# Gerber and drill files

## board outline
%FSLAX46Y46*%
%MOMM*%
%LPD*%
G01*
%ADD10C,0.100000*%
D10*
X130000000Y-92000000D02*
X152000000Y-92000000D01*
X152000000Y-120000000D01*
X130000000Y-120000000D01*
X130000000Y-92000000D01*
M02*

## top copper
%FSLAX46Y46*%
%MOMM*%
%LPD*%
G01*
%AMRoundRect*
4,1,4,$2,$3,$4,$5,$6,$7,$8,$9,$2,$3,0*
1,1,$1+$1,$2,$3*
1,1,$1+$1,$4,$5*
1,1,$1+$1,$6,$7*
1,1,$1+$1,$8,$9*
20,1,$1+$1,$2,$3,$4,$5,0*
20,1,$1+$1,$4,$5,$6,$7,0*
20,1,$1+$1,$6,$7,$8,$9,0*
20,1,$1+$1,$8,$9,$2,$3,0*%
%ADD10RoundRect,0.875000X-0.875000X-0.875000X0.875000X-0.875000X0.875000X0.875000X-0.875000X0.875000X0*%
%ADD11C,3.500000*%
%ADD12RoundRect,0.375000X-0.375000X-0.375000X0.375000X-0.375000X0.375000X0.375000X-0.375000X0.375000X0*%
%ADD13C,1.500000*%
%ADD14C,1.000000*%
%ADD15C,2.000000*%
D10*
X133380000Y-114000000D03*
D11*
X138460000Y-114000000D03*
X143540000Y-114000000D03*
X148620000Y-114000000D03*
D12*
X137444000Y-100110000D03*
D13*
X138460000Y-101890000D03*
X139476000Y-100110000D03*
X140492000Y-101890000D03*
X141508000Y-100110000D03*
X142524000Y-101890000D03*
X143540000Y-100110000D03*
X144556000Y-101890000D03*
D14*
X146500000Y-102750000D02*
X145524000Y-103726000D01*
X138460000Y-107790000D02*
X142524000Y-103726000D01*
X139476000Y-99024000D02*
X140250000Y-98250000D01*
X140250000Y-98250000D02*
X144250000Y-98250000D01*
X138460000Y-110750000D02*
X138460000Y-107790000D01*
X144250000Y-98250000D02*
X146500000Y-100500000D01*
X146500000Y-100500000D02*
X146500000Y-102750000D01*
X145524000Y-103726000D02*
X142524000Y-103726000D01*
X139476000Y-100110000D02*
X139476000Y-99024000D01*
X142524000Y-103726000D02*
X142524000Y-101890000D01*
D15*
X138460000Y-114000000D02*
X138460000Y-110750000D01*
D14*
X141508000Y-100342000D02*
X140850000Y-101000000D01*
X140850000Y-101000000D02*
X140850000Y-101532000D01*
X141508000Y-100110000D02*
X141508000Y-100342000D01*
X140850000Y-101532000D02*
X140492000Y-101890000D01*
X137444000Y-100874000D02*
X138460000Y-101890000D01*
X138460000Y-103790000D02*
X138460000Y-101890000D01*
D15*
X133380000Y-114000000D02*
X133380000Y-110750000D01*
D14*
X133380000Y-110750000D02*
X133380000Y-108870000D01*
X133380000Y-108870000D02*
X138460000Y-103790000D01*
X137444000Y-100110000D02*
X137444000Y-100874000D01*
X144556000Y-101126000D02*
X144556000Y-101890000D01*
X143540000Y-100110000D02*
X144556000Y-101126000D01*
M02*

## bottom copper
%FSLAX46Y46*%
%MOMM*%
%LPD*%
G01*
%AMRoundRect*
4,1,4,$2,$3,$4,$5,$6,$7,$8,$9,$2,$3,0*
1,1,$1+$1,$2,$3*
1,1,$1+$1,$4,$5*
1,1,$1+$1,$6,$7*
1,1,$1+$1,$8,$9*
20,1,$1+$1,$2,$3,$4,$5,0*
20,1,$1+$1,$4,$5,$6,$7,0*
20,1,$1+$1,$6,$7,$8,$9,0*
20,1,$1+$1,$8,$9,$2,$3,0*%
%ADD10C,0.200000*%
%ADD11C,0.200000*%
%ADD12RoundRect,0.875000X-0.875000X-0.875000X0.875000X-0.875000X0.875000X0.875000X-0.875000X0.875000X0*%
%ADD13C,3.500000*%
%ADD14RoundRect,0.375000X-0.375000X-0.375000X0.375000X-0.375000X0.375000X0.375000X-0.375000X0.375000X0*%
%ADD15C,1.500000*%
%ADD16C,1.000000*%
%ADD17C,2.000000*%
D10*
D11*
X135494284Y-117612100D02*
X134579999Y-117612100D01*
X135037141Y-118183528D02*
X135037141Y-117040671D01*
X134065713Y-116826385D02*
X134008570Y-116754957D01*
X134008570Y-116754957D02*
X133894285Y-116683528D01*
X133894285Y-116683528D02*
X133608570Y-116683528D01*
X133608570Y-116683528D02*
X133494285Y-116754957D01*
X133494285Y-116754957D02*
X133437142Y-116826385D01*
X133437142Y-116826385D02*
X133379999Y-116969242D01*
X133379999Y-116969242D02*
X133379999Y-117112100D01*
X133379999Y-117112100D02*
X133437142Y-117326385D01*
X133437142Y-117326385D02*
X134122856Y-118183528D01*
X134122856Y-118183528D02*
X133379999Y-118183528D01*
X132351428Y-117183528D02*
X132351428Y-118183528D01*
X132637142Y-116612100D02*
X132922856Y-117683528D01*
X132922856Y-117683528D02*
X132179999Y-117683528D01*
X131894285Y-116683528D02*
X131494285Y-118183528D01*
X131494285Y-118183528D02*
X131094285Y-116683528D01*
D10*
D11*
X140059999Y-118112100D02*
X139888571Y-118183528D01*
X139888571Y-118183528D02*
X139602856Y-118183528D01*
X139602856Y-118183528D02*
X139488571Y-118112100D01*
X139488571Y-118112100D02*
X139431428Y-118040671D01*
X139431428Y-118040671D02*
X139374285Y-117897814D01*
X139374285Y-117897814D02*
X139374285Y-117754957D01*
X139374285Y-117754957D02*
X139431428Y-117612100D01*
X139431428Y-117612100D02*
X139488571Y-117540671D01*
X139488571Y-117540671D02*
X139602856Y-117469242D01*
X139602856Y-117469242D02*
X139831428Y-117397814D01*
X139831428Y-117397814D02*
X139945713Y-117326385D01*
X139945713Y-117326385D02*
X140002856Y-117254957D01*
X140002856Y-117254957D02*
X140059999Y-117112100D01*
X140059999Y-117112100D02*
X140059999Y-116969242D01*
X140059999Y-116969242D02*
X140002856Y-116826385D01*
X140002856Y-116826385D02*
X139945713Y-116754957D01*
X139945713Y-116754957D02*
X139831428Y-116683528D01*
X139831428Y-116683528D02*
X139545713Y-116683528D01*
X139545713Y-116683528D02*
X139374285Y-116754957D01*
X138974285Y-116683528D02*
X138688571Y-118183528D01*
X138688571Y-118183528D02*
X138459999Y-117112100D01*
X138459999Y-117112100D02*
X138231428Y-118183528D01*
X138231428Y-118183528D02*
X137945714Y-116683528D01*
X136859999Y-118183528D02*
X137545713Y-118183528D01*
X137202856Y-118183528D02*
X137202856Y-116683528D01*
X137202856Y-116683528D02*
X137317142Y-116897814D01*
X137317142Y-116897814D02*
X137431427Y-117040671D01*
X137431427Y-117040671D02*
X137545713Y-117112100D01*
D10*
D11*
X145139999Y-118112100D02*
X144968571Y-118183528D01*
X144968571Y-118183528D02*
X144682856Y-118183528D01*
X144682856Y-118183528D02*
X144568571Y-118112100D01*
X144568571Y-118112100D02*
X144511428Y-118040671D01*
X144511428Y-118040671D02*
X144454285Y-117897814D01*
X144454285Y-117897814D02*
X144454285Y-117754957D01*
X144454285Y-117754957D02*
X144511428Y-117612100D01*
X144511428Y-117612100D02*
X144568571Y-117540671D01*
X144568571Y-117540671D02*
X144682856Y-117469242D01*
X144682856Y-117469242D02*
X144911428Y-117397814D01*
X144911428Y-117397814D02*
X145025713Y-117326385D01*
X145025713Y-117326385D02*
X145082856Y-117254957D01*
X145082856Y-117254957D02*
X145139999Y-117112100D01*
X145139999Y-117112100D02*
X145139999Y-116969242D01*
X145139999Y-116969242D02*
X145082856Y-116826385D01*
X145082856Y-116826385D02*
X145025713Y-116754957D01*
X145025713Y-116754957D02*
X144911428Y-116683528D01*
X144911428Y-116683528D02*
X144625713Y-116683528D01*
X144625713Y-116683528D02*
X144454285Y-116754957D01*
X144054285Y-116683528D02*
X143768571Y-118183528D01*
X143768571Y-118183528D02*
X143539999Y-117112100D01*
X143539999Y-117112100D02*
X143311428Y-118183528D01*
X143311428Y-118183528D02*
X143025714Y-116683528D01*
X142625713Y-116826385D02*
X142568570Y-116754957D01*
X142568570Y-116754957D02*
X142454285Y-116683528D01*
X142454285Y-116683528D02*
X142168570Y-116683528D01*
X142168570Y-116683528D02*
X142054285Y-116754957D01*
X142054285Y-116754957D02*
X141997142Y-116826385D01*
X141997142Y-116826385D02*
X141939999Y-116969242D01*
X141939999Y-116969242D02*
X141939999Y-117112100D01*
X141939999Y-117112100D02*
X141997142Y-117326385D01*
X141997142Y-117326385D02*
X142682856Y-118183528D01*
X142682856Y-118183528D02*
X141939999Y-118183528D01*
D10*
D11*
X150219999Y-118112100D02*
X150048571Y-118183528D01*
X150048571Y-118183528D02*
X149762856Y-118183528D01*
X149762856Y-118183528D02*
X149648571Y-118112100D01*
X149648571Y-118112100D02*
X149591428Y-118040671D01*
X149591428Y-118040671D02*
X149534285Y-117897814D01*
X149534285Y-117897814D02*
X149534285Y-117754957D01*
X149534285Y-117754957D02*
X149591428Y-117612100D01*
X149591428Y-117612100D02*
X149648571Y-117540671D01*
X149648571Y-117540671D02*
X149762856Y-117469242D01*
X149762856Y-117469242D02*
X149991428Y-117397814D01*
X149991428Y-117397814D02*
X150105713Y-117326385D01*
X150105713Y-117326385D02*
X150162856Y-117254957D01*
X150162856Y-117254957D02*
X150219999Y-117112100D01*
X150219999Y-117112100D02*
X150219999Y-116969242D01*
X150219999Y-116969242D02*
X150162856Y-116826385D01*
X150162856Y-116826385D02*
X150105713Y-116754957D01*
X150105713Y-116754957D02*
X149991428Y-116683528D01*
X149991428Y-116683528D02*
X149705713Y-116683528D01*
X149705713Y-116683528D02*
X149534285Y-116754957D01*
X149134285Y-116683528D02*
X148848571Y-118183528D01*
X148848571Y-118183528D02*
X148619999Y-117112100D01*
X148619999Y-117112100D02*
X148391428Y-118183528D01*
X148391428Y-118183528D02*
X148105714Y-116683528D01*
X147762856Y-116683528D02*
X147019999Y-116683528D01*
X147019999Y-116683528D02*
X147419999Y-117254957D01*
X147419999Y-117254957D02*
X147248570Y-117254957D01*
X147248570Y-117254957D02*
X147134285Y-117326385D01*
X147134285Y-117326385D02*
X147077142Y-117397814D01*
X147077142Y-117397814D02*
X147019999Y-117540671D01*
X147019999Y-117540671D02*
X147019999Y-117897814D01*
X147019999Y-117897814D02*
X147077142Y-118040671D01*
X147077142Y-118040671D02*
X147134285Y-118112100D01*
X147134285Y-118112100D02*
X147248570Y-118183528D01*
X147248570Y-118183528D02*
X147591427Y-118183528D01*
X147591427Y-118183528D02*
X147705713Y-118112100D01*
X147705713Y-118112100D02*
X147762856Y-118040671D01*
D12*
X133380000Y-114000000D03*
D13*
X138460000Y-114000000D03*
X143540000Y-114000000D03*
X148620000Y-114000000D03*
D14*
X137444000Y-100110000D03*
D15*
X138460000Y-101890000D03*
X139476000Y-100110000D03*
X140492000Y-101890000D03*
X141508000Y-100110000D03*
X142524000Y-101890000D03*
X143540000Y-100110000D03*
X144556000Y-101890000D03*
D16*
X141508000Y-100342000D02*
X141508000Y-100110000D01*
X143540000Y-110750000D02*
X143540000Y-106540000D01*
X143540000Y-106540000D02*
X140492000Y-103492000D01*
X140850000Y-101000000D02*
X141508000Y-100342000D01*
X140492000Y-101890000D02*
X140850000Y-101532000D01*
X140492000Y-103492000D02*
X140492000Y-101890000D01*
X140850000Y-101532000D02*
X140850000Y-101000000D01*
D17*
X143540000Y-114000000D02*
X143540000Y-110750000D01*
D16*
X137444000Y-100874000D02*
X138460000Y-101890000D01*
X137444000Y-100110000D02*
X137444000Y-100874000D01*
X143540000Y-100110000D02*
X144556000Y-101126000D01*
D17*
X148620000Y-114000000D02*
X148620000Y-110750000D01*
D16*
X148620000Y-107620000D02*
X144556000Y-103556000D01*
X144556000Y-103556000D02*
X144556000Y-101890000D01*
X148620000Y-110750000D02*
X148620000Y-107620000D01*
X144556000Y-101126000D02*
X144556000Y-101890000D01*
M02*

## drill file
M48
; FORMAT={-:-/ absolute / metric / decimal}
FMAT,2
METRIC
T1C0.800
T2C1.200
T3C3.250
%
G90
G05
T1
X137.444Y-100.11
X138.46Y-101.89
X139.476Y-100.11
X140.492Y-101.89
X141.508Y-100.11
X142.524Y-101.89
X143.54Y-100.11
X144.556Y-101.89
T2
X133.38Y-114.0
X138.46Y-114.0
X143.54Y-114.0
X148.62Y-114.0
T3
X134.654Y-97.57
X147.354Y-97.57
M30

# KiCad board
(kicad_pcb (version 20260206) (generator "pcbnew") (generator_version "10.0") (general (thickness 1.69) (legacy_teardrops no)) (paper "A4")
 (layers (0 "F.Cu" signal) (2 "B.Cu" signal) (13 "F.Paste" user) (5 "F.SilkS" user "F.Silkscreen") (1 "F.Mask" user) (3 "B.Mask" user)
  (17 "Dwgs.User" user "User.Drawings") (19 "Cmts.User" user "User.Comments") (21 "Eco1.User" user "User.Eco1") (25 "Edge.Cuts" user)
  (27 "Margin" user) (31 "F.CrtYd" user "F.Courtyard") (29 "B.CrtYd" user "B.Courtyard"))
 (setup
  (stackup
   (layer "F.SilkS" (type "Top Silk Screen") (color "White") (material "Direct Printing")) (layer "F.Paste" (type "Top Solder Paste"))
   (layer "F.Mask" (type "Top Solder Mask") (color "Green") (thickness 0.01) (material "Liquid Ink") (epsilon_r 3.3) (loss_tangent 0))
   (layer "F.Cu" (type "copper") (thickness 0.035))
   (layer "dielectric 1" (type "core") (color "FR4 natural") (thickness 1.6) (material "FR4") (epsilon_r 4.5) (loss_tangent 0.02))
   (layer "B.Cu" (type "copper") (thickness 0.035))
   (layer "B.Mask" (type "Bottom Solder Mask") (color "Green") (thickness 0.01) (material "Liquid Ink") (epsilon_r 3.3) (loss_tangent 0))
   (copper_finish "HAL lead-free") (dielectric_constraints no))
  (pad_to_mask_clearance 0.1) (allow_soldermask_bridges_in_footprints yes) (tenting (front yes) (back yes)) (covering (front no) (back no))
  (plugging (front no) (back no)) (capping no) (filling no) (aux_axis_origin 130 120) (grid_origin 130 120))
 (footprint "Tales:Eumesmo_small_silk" (layer "F.Cu") (at 148.5 100 90)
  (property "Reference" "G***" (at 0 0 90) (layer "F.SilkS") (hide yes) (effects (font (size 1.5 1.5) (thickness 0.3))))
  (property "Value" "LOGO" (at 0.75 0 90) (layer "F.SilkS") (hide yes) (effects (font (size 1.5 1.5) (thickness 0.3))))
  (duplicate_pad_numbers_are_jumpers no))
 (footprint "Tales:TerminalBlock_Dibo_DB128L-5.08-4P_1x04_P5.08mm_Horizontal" (layer "F.Cu") (at 141 114)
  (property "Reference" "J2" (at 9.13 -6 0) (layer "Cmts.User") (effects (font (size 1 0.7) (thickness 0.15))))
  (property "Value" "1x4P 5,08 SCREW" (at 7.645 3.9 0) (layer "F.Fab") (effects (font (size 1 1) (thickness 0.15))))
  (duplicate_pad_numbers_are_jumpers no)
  (pad "1" thru_hole roundrect (at -7.62 0) (size 3.5 3.5) (drill 1.2) (layers "*.Cu" "*.Mask") (remove_unused_layers no)
   (roundrect_rratio 0.25) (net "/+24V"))
  (pad "2" thru_hole circle (at -2.54 0) (size 3.5 3.5) (drill 1.2) (layers "*.Cu" "*.Mask") (remove_unused_layers no) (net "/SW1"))
  (pad "3" thru_hole circle (at 2.54 0) (size 3.5 3.5) (drill 1.2) (layers "*.Cu" "*.Mask") (remove_unused_layers no) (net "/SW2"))
  (pad "4" thru_hole circle (at 7.62 0) (size 3.5 3.5) (drill 1.2) (layers "*.Cu" "*.Mask") (remove_unused_layers no) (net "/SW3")))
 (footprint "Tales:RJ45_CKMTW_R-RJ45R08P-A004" (layer "F.Cu") (at 141 101 180)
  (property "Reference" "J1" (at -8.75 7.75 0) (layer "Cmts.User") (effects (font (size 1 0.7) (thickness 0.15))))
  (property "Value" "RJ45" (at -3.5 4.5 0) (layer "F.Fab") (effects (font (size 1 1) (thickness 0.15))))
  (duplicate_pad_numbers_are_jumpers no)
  (pad "" np_thru_hole circle (at -6.354 3.43) (size 3.25 3.25) (drill 3.25) (layers "*.Cu" "*.Mask"))
  (pad "" np_thru_hole circle (at 6.346 3.43) (size 3.25 3.25) (drill 3.25) (layers "*.Cu" "*.Mask"))
  (pad "1" thru_hole roundrect (at 3.556 0.89) (size 1.5 1.5) (drill 0.8) (layers "*.Cu" "*.Mask") (remove_unused_layers no)
   (roundrect_rratio 0.25) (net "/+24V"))
  (pad "2" thru_hole circle (at 2.54 -0.89) (size 1.5 1.5) (drill 0.8) (layers "*.Cu" "*.Mask") (remove_unused_layers no) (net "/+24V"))
  (pad "3" thru_hole circle (at 1.524 0.89) (size 1.5 1.5) (drill 0.8) (layers "*.Cu" "*.Mask") (remove_unused_layers no) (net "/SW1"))
  (pad "4" thru_hole circle (at 0.508 -0.89) (size 1.5 1.5) (drill 0.8) (layers "*.Cu" "*.Mask") (remove_unused_layers no) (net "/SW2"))
  (pad "5" thru_hole circle (at -0.508 0.89) (size 1.5 1.5) (drill 0.8) (layers "*.Cu" "*.Mask") (remove_unused_layers no) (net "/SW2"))
  (pad "6" thru_hole circle (at -1.524 -0.89) (size 1.5 1.5) (drill 0.8) (layers "*.Cu" "*.Mask") (remove_unused_layers no) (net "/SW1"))
  (pad "7" thru_hole circle (at -2.54 0.89) (size 1.5 1.5) (drill 0.8) (layers "*.Cu" "*.Mask") (remove_unused_layers no) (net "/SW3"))
  (pad "8" thru_hole circle (at -3.556 -0.89) (size 1.5 1.5) (drill 0.8) (layers "*.Cu" "*.Mask") (remove_unused_layers no) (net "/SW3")))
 (gr_rect (start 130 92) (end 152 120) (stroke (width 0.1) (type default)) (fill no) (layer "Edge.Cuts"))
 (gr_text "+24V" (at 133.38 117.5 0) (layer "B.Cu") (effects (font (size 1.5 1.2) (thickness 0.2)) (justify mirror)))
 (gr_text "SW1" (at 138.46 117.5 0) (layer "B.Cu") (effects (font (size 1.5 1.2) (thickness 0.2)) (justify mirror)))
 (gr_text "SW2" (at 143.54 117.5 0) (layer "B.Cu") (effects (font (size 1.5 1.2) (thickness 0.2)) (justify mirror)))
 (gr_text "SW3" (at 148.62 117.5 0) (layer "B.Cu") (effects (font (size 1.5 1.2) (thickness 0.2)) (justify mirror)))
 (segment (start 146.5 102.75) (end 145.524 103.726) (width 1) (layer "F.Cu") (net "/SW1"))
 (segment (start 138.46 107.79) (end 142.524 103.726) (width 1) (layer "F.Cu") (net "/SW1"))
 (segment (start 139.476 99.024) (end 140.25 98.25) (width 1) (layer "F.Cu") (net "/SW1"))
 (segment (start 140.25 98.25) (end 144.25 98.25) (width 1) (layer "F.Cu") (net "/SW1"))
 (segment (start 138.46 110.75) (end 138.46 107.79) (width 1) (layer "F.Cu") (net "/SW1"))
 (segment (start 144.25 98.25) (end 146.5 100.5) (width 1) (layer "F.Cu") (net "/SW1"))
 (segment (start 146.5 100.5) (end 146.5 102.75) (width 1) (layer "F.Cu") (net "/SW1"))
 (segment (start 145.524 103.726) (end 142.524 103.726) (width 1) (layer "F.Cu") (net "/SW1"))
 (segment (start 139.476 100.11) (end 139.476 99.024) (width 1) (layer "F.Cu") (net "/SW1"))
 (segment (start 142.524 103.726) (end 142.524 101.89) (width 1) (layer "F.Cu") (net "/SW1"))
 (segment (start 138.46 114) (end 138.46 110.75) (width 2) (layer "F.Cu") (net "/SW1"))
 (segment (start 141.508 100.342) (end 140.85 101) (width 1) (layer "F.Cu") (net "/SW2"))
 (segment (start 140.85 101) (end 140.85 101.532) (width 1) (layer "F.Cu") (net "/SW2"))
 (segment (start 141.508 100.11) (end 141.508 100.342) (width 1) (layer "F.Cu") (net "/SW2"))
 (segment (start 140.85 101.532) (end 140.492 101.89) (width 1) (layer "F.Cu") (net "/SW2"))
 (segment (start 141.508 100.342) (end 141.508 100.11) (width 1) (layer "B.Cu") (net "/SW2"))
 (segment (start 143.54 110.75) (end 143.54 106.54) (width 1) (layer "B.Cu") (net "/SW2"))
 (segment (start 143.54 106.54) (end 140.492 103.492) (width 1) (layer "B.Cu") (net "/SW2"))
 (segment (start 140.85 101) (end 141.508 100.342) (width 1) (layer "B.Cu") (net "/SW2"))
 (segment (start 140.492 101.89) (end 140.85 101.532) (width 1) (layer "B.Cu") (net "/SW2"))
 (segment (start 140.492 103.492) (end 140.492 101.89) (width 1) (layer "B.Cu") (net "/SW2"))
 (segment (start 140.85 101.532) (end 140.85 101) (width 1) (layer "B.Cu") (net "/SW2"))
 (segment (start 143.54 114) (end 143.54 110.75) (width 2) (layer "B.Cu") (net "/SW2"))
 (segment (start 137.444 100.874) (end 138.46 101.89) (width 1) (layer "F.Cu") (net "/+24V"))
 (segment (start 138.46 103.79) (end 138.46 101.89) (width 1) (layer "F.Cu") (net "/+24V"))
 (segment (start 133.38 114) (end 133.38 110.75) (width 2) (layer "F.Cu") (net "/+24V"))
 (segment (start 133.38 110.75) (end 133.38 108.87) (width 1) (layer "F.Cu") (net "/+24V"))
 (segment (start 133.38 108.87) (end 138.46 103.79) (width 1) (layer "F.Cu") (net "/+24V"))
 (segment (start 137.444 100.11) (end 137.444 100.874) (width 1) (layer "F.Cu") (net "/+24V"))
 (segment (start 137.444 100.874) (end 138.46 101.89) (width 1) (layer "B.Cu") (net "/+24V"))
 (segment (start 137.444 100.11) (end 137.444 100.874) (width 1) (layer "B.Cu") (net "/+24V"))
 (segment (start 144.556 101.126) (end 144.556 101.89) (width 1) (layer "F.Cu") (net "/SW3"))
 (segment (start 143.54 100.11) (end 144.556 101.126) (width 1) (layer "F.Cu") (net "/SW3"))
 (segment (start 143.54 100.11) (end 144.556 101.126) (width 1) (layer "B.Cu") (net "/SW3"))
 (segment (start 148.62 114) (end 148.62 110.75) (width 2) (layer "B.Cu") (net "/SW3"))
 (segment (start 148.62 107.62) (end 144.556 103.556) (width 1) (layer "B.Cu") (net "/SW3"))
 (segment (start 144.556 103.556) (end 144.556 101.89) (width 1) (layer "B.Cu") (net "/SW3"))
 (segment (start 148.62 110.75) (end 148.62 107.62) (width 1) (layer "B.Cu") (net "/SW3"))
 (segment (start 144.556 101.126) (end 144.556 101.89) (width 1) (layer "B.Cu") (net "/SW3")))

